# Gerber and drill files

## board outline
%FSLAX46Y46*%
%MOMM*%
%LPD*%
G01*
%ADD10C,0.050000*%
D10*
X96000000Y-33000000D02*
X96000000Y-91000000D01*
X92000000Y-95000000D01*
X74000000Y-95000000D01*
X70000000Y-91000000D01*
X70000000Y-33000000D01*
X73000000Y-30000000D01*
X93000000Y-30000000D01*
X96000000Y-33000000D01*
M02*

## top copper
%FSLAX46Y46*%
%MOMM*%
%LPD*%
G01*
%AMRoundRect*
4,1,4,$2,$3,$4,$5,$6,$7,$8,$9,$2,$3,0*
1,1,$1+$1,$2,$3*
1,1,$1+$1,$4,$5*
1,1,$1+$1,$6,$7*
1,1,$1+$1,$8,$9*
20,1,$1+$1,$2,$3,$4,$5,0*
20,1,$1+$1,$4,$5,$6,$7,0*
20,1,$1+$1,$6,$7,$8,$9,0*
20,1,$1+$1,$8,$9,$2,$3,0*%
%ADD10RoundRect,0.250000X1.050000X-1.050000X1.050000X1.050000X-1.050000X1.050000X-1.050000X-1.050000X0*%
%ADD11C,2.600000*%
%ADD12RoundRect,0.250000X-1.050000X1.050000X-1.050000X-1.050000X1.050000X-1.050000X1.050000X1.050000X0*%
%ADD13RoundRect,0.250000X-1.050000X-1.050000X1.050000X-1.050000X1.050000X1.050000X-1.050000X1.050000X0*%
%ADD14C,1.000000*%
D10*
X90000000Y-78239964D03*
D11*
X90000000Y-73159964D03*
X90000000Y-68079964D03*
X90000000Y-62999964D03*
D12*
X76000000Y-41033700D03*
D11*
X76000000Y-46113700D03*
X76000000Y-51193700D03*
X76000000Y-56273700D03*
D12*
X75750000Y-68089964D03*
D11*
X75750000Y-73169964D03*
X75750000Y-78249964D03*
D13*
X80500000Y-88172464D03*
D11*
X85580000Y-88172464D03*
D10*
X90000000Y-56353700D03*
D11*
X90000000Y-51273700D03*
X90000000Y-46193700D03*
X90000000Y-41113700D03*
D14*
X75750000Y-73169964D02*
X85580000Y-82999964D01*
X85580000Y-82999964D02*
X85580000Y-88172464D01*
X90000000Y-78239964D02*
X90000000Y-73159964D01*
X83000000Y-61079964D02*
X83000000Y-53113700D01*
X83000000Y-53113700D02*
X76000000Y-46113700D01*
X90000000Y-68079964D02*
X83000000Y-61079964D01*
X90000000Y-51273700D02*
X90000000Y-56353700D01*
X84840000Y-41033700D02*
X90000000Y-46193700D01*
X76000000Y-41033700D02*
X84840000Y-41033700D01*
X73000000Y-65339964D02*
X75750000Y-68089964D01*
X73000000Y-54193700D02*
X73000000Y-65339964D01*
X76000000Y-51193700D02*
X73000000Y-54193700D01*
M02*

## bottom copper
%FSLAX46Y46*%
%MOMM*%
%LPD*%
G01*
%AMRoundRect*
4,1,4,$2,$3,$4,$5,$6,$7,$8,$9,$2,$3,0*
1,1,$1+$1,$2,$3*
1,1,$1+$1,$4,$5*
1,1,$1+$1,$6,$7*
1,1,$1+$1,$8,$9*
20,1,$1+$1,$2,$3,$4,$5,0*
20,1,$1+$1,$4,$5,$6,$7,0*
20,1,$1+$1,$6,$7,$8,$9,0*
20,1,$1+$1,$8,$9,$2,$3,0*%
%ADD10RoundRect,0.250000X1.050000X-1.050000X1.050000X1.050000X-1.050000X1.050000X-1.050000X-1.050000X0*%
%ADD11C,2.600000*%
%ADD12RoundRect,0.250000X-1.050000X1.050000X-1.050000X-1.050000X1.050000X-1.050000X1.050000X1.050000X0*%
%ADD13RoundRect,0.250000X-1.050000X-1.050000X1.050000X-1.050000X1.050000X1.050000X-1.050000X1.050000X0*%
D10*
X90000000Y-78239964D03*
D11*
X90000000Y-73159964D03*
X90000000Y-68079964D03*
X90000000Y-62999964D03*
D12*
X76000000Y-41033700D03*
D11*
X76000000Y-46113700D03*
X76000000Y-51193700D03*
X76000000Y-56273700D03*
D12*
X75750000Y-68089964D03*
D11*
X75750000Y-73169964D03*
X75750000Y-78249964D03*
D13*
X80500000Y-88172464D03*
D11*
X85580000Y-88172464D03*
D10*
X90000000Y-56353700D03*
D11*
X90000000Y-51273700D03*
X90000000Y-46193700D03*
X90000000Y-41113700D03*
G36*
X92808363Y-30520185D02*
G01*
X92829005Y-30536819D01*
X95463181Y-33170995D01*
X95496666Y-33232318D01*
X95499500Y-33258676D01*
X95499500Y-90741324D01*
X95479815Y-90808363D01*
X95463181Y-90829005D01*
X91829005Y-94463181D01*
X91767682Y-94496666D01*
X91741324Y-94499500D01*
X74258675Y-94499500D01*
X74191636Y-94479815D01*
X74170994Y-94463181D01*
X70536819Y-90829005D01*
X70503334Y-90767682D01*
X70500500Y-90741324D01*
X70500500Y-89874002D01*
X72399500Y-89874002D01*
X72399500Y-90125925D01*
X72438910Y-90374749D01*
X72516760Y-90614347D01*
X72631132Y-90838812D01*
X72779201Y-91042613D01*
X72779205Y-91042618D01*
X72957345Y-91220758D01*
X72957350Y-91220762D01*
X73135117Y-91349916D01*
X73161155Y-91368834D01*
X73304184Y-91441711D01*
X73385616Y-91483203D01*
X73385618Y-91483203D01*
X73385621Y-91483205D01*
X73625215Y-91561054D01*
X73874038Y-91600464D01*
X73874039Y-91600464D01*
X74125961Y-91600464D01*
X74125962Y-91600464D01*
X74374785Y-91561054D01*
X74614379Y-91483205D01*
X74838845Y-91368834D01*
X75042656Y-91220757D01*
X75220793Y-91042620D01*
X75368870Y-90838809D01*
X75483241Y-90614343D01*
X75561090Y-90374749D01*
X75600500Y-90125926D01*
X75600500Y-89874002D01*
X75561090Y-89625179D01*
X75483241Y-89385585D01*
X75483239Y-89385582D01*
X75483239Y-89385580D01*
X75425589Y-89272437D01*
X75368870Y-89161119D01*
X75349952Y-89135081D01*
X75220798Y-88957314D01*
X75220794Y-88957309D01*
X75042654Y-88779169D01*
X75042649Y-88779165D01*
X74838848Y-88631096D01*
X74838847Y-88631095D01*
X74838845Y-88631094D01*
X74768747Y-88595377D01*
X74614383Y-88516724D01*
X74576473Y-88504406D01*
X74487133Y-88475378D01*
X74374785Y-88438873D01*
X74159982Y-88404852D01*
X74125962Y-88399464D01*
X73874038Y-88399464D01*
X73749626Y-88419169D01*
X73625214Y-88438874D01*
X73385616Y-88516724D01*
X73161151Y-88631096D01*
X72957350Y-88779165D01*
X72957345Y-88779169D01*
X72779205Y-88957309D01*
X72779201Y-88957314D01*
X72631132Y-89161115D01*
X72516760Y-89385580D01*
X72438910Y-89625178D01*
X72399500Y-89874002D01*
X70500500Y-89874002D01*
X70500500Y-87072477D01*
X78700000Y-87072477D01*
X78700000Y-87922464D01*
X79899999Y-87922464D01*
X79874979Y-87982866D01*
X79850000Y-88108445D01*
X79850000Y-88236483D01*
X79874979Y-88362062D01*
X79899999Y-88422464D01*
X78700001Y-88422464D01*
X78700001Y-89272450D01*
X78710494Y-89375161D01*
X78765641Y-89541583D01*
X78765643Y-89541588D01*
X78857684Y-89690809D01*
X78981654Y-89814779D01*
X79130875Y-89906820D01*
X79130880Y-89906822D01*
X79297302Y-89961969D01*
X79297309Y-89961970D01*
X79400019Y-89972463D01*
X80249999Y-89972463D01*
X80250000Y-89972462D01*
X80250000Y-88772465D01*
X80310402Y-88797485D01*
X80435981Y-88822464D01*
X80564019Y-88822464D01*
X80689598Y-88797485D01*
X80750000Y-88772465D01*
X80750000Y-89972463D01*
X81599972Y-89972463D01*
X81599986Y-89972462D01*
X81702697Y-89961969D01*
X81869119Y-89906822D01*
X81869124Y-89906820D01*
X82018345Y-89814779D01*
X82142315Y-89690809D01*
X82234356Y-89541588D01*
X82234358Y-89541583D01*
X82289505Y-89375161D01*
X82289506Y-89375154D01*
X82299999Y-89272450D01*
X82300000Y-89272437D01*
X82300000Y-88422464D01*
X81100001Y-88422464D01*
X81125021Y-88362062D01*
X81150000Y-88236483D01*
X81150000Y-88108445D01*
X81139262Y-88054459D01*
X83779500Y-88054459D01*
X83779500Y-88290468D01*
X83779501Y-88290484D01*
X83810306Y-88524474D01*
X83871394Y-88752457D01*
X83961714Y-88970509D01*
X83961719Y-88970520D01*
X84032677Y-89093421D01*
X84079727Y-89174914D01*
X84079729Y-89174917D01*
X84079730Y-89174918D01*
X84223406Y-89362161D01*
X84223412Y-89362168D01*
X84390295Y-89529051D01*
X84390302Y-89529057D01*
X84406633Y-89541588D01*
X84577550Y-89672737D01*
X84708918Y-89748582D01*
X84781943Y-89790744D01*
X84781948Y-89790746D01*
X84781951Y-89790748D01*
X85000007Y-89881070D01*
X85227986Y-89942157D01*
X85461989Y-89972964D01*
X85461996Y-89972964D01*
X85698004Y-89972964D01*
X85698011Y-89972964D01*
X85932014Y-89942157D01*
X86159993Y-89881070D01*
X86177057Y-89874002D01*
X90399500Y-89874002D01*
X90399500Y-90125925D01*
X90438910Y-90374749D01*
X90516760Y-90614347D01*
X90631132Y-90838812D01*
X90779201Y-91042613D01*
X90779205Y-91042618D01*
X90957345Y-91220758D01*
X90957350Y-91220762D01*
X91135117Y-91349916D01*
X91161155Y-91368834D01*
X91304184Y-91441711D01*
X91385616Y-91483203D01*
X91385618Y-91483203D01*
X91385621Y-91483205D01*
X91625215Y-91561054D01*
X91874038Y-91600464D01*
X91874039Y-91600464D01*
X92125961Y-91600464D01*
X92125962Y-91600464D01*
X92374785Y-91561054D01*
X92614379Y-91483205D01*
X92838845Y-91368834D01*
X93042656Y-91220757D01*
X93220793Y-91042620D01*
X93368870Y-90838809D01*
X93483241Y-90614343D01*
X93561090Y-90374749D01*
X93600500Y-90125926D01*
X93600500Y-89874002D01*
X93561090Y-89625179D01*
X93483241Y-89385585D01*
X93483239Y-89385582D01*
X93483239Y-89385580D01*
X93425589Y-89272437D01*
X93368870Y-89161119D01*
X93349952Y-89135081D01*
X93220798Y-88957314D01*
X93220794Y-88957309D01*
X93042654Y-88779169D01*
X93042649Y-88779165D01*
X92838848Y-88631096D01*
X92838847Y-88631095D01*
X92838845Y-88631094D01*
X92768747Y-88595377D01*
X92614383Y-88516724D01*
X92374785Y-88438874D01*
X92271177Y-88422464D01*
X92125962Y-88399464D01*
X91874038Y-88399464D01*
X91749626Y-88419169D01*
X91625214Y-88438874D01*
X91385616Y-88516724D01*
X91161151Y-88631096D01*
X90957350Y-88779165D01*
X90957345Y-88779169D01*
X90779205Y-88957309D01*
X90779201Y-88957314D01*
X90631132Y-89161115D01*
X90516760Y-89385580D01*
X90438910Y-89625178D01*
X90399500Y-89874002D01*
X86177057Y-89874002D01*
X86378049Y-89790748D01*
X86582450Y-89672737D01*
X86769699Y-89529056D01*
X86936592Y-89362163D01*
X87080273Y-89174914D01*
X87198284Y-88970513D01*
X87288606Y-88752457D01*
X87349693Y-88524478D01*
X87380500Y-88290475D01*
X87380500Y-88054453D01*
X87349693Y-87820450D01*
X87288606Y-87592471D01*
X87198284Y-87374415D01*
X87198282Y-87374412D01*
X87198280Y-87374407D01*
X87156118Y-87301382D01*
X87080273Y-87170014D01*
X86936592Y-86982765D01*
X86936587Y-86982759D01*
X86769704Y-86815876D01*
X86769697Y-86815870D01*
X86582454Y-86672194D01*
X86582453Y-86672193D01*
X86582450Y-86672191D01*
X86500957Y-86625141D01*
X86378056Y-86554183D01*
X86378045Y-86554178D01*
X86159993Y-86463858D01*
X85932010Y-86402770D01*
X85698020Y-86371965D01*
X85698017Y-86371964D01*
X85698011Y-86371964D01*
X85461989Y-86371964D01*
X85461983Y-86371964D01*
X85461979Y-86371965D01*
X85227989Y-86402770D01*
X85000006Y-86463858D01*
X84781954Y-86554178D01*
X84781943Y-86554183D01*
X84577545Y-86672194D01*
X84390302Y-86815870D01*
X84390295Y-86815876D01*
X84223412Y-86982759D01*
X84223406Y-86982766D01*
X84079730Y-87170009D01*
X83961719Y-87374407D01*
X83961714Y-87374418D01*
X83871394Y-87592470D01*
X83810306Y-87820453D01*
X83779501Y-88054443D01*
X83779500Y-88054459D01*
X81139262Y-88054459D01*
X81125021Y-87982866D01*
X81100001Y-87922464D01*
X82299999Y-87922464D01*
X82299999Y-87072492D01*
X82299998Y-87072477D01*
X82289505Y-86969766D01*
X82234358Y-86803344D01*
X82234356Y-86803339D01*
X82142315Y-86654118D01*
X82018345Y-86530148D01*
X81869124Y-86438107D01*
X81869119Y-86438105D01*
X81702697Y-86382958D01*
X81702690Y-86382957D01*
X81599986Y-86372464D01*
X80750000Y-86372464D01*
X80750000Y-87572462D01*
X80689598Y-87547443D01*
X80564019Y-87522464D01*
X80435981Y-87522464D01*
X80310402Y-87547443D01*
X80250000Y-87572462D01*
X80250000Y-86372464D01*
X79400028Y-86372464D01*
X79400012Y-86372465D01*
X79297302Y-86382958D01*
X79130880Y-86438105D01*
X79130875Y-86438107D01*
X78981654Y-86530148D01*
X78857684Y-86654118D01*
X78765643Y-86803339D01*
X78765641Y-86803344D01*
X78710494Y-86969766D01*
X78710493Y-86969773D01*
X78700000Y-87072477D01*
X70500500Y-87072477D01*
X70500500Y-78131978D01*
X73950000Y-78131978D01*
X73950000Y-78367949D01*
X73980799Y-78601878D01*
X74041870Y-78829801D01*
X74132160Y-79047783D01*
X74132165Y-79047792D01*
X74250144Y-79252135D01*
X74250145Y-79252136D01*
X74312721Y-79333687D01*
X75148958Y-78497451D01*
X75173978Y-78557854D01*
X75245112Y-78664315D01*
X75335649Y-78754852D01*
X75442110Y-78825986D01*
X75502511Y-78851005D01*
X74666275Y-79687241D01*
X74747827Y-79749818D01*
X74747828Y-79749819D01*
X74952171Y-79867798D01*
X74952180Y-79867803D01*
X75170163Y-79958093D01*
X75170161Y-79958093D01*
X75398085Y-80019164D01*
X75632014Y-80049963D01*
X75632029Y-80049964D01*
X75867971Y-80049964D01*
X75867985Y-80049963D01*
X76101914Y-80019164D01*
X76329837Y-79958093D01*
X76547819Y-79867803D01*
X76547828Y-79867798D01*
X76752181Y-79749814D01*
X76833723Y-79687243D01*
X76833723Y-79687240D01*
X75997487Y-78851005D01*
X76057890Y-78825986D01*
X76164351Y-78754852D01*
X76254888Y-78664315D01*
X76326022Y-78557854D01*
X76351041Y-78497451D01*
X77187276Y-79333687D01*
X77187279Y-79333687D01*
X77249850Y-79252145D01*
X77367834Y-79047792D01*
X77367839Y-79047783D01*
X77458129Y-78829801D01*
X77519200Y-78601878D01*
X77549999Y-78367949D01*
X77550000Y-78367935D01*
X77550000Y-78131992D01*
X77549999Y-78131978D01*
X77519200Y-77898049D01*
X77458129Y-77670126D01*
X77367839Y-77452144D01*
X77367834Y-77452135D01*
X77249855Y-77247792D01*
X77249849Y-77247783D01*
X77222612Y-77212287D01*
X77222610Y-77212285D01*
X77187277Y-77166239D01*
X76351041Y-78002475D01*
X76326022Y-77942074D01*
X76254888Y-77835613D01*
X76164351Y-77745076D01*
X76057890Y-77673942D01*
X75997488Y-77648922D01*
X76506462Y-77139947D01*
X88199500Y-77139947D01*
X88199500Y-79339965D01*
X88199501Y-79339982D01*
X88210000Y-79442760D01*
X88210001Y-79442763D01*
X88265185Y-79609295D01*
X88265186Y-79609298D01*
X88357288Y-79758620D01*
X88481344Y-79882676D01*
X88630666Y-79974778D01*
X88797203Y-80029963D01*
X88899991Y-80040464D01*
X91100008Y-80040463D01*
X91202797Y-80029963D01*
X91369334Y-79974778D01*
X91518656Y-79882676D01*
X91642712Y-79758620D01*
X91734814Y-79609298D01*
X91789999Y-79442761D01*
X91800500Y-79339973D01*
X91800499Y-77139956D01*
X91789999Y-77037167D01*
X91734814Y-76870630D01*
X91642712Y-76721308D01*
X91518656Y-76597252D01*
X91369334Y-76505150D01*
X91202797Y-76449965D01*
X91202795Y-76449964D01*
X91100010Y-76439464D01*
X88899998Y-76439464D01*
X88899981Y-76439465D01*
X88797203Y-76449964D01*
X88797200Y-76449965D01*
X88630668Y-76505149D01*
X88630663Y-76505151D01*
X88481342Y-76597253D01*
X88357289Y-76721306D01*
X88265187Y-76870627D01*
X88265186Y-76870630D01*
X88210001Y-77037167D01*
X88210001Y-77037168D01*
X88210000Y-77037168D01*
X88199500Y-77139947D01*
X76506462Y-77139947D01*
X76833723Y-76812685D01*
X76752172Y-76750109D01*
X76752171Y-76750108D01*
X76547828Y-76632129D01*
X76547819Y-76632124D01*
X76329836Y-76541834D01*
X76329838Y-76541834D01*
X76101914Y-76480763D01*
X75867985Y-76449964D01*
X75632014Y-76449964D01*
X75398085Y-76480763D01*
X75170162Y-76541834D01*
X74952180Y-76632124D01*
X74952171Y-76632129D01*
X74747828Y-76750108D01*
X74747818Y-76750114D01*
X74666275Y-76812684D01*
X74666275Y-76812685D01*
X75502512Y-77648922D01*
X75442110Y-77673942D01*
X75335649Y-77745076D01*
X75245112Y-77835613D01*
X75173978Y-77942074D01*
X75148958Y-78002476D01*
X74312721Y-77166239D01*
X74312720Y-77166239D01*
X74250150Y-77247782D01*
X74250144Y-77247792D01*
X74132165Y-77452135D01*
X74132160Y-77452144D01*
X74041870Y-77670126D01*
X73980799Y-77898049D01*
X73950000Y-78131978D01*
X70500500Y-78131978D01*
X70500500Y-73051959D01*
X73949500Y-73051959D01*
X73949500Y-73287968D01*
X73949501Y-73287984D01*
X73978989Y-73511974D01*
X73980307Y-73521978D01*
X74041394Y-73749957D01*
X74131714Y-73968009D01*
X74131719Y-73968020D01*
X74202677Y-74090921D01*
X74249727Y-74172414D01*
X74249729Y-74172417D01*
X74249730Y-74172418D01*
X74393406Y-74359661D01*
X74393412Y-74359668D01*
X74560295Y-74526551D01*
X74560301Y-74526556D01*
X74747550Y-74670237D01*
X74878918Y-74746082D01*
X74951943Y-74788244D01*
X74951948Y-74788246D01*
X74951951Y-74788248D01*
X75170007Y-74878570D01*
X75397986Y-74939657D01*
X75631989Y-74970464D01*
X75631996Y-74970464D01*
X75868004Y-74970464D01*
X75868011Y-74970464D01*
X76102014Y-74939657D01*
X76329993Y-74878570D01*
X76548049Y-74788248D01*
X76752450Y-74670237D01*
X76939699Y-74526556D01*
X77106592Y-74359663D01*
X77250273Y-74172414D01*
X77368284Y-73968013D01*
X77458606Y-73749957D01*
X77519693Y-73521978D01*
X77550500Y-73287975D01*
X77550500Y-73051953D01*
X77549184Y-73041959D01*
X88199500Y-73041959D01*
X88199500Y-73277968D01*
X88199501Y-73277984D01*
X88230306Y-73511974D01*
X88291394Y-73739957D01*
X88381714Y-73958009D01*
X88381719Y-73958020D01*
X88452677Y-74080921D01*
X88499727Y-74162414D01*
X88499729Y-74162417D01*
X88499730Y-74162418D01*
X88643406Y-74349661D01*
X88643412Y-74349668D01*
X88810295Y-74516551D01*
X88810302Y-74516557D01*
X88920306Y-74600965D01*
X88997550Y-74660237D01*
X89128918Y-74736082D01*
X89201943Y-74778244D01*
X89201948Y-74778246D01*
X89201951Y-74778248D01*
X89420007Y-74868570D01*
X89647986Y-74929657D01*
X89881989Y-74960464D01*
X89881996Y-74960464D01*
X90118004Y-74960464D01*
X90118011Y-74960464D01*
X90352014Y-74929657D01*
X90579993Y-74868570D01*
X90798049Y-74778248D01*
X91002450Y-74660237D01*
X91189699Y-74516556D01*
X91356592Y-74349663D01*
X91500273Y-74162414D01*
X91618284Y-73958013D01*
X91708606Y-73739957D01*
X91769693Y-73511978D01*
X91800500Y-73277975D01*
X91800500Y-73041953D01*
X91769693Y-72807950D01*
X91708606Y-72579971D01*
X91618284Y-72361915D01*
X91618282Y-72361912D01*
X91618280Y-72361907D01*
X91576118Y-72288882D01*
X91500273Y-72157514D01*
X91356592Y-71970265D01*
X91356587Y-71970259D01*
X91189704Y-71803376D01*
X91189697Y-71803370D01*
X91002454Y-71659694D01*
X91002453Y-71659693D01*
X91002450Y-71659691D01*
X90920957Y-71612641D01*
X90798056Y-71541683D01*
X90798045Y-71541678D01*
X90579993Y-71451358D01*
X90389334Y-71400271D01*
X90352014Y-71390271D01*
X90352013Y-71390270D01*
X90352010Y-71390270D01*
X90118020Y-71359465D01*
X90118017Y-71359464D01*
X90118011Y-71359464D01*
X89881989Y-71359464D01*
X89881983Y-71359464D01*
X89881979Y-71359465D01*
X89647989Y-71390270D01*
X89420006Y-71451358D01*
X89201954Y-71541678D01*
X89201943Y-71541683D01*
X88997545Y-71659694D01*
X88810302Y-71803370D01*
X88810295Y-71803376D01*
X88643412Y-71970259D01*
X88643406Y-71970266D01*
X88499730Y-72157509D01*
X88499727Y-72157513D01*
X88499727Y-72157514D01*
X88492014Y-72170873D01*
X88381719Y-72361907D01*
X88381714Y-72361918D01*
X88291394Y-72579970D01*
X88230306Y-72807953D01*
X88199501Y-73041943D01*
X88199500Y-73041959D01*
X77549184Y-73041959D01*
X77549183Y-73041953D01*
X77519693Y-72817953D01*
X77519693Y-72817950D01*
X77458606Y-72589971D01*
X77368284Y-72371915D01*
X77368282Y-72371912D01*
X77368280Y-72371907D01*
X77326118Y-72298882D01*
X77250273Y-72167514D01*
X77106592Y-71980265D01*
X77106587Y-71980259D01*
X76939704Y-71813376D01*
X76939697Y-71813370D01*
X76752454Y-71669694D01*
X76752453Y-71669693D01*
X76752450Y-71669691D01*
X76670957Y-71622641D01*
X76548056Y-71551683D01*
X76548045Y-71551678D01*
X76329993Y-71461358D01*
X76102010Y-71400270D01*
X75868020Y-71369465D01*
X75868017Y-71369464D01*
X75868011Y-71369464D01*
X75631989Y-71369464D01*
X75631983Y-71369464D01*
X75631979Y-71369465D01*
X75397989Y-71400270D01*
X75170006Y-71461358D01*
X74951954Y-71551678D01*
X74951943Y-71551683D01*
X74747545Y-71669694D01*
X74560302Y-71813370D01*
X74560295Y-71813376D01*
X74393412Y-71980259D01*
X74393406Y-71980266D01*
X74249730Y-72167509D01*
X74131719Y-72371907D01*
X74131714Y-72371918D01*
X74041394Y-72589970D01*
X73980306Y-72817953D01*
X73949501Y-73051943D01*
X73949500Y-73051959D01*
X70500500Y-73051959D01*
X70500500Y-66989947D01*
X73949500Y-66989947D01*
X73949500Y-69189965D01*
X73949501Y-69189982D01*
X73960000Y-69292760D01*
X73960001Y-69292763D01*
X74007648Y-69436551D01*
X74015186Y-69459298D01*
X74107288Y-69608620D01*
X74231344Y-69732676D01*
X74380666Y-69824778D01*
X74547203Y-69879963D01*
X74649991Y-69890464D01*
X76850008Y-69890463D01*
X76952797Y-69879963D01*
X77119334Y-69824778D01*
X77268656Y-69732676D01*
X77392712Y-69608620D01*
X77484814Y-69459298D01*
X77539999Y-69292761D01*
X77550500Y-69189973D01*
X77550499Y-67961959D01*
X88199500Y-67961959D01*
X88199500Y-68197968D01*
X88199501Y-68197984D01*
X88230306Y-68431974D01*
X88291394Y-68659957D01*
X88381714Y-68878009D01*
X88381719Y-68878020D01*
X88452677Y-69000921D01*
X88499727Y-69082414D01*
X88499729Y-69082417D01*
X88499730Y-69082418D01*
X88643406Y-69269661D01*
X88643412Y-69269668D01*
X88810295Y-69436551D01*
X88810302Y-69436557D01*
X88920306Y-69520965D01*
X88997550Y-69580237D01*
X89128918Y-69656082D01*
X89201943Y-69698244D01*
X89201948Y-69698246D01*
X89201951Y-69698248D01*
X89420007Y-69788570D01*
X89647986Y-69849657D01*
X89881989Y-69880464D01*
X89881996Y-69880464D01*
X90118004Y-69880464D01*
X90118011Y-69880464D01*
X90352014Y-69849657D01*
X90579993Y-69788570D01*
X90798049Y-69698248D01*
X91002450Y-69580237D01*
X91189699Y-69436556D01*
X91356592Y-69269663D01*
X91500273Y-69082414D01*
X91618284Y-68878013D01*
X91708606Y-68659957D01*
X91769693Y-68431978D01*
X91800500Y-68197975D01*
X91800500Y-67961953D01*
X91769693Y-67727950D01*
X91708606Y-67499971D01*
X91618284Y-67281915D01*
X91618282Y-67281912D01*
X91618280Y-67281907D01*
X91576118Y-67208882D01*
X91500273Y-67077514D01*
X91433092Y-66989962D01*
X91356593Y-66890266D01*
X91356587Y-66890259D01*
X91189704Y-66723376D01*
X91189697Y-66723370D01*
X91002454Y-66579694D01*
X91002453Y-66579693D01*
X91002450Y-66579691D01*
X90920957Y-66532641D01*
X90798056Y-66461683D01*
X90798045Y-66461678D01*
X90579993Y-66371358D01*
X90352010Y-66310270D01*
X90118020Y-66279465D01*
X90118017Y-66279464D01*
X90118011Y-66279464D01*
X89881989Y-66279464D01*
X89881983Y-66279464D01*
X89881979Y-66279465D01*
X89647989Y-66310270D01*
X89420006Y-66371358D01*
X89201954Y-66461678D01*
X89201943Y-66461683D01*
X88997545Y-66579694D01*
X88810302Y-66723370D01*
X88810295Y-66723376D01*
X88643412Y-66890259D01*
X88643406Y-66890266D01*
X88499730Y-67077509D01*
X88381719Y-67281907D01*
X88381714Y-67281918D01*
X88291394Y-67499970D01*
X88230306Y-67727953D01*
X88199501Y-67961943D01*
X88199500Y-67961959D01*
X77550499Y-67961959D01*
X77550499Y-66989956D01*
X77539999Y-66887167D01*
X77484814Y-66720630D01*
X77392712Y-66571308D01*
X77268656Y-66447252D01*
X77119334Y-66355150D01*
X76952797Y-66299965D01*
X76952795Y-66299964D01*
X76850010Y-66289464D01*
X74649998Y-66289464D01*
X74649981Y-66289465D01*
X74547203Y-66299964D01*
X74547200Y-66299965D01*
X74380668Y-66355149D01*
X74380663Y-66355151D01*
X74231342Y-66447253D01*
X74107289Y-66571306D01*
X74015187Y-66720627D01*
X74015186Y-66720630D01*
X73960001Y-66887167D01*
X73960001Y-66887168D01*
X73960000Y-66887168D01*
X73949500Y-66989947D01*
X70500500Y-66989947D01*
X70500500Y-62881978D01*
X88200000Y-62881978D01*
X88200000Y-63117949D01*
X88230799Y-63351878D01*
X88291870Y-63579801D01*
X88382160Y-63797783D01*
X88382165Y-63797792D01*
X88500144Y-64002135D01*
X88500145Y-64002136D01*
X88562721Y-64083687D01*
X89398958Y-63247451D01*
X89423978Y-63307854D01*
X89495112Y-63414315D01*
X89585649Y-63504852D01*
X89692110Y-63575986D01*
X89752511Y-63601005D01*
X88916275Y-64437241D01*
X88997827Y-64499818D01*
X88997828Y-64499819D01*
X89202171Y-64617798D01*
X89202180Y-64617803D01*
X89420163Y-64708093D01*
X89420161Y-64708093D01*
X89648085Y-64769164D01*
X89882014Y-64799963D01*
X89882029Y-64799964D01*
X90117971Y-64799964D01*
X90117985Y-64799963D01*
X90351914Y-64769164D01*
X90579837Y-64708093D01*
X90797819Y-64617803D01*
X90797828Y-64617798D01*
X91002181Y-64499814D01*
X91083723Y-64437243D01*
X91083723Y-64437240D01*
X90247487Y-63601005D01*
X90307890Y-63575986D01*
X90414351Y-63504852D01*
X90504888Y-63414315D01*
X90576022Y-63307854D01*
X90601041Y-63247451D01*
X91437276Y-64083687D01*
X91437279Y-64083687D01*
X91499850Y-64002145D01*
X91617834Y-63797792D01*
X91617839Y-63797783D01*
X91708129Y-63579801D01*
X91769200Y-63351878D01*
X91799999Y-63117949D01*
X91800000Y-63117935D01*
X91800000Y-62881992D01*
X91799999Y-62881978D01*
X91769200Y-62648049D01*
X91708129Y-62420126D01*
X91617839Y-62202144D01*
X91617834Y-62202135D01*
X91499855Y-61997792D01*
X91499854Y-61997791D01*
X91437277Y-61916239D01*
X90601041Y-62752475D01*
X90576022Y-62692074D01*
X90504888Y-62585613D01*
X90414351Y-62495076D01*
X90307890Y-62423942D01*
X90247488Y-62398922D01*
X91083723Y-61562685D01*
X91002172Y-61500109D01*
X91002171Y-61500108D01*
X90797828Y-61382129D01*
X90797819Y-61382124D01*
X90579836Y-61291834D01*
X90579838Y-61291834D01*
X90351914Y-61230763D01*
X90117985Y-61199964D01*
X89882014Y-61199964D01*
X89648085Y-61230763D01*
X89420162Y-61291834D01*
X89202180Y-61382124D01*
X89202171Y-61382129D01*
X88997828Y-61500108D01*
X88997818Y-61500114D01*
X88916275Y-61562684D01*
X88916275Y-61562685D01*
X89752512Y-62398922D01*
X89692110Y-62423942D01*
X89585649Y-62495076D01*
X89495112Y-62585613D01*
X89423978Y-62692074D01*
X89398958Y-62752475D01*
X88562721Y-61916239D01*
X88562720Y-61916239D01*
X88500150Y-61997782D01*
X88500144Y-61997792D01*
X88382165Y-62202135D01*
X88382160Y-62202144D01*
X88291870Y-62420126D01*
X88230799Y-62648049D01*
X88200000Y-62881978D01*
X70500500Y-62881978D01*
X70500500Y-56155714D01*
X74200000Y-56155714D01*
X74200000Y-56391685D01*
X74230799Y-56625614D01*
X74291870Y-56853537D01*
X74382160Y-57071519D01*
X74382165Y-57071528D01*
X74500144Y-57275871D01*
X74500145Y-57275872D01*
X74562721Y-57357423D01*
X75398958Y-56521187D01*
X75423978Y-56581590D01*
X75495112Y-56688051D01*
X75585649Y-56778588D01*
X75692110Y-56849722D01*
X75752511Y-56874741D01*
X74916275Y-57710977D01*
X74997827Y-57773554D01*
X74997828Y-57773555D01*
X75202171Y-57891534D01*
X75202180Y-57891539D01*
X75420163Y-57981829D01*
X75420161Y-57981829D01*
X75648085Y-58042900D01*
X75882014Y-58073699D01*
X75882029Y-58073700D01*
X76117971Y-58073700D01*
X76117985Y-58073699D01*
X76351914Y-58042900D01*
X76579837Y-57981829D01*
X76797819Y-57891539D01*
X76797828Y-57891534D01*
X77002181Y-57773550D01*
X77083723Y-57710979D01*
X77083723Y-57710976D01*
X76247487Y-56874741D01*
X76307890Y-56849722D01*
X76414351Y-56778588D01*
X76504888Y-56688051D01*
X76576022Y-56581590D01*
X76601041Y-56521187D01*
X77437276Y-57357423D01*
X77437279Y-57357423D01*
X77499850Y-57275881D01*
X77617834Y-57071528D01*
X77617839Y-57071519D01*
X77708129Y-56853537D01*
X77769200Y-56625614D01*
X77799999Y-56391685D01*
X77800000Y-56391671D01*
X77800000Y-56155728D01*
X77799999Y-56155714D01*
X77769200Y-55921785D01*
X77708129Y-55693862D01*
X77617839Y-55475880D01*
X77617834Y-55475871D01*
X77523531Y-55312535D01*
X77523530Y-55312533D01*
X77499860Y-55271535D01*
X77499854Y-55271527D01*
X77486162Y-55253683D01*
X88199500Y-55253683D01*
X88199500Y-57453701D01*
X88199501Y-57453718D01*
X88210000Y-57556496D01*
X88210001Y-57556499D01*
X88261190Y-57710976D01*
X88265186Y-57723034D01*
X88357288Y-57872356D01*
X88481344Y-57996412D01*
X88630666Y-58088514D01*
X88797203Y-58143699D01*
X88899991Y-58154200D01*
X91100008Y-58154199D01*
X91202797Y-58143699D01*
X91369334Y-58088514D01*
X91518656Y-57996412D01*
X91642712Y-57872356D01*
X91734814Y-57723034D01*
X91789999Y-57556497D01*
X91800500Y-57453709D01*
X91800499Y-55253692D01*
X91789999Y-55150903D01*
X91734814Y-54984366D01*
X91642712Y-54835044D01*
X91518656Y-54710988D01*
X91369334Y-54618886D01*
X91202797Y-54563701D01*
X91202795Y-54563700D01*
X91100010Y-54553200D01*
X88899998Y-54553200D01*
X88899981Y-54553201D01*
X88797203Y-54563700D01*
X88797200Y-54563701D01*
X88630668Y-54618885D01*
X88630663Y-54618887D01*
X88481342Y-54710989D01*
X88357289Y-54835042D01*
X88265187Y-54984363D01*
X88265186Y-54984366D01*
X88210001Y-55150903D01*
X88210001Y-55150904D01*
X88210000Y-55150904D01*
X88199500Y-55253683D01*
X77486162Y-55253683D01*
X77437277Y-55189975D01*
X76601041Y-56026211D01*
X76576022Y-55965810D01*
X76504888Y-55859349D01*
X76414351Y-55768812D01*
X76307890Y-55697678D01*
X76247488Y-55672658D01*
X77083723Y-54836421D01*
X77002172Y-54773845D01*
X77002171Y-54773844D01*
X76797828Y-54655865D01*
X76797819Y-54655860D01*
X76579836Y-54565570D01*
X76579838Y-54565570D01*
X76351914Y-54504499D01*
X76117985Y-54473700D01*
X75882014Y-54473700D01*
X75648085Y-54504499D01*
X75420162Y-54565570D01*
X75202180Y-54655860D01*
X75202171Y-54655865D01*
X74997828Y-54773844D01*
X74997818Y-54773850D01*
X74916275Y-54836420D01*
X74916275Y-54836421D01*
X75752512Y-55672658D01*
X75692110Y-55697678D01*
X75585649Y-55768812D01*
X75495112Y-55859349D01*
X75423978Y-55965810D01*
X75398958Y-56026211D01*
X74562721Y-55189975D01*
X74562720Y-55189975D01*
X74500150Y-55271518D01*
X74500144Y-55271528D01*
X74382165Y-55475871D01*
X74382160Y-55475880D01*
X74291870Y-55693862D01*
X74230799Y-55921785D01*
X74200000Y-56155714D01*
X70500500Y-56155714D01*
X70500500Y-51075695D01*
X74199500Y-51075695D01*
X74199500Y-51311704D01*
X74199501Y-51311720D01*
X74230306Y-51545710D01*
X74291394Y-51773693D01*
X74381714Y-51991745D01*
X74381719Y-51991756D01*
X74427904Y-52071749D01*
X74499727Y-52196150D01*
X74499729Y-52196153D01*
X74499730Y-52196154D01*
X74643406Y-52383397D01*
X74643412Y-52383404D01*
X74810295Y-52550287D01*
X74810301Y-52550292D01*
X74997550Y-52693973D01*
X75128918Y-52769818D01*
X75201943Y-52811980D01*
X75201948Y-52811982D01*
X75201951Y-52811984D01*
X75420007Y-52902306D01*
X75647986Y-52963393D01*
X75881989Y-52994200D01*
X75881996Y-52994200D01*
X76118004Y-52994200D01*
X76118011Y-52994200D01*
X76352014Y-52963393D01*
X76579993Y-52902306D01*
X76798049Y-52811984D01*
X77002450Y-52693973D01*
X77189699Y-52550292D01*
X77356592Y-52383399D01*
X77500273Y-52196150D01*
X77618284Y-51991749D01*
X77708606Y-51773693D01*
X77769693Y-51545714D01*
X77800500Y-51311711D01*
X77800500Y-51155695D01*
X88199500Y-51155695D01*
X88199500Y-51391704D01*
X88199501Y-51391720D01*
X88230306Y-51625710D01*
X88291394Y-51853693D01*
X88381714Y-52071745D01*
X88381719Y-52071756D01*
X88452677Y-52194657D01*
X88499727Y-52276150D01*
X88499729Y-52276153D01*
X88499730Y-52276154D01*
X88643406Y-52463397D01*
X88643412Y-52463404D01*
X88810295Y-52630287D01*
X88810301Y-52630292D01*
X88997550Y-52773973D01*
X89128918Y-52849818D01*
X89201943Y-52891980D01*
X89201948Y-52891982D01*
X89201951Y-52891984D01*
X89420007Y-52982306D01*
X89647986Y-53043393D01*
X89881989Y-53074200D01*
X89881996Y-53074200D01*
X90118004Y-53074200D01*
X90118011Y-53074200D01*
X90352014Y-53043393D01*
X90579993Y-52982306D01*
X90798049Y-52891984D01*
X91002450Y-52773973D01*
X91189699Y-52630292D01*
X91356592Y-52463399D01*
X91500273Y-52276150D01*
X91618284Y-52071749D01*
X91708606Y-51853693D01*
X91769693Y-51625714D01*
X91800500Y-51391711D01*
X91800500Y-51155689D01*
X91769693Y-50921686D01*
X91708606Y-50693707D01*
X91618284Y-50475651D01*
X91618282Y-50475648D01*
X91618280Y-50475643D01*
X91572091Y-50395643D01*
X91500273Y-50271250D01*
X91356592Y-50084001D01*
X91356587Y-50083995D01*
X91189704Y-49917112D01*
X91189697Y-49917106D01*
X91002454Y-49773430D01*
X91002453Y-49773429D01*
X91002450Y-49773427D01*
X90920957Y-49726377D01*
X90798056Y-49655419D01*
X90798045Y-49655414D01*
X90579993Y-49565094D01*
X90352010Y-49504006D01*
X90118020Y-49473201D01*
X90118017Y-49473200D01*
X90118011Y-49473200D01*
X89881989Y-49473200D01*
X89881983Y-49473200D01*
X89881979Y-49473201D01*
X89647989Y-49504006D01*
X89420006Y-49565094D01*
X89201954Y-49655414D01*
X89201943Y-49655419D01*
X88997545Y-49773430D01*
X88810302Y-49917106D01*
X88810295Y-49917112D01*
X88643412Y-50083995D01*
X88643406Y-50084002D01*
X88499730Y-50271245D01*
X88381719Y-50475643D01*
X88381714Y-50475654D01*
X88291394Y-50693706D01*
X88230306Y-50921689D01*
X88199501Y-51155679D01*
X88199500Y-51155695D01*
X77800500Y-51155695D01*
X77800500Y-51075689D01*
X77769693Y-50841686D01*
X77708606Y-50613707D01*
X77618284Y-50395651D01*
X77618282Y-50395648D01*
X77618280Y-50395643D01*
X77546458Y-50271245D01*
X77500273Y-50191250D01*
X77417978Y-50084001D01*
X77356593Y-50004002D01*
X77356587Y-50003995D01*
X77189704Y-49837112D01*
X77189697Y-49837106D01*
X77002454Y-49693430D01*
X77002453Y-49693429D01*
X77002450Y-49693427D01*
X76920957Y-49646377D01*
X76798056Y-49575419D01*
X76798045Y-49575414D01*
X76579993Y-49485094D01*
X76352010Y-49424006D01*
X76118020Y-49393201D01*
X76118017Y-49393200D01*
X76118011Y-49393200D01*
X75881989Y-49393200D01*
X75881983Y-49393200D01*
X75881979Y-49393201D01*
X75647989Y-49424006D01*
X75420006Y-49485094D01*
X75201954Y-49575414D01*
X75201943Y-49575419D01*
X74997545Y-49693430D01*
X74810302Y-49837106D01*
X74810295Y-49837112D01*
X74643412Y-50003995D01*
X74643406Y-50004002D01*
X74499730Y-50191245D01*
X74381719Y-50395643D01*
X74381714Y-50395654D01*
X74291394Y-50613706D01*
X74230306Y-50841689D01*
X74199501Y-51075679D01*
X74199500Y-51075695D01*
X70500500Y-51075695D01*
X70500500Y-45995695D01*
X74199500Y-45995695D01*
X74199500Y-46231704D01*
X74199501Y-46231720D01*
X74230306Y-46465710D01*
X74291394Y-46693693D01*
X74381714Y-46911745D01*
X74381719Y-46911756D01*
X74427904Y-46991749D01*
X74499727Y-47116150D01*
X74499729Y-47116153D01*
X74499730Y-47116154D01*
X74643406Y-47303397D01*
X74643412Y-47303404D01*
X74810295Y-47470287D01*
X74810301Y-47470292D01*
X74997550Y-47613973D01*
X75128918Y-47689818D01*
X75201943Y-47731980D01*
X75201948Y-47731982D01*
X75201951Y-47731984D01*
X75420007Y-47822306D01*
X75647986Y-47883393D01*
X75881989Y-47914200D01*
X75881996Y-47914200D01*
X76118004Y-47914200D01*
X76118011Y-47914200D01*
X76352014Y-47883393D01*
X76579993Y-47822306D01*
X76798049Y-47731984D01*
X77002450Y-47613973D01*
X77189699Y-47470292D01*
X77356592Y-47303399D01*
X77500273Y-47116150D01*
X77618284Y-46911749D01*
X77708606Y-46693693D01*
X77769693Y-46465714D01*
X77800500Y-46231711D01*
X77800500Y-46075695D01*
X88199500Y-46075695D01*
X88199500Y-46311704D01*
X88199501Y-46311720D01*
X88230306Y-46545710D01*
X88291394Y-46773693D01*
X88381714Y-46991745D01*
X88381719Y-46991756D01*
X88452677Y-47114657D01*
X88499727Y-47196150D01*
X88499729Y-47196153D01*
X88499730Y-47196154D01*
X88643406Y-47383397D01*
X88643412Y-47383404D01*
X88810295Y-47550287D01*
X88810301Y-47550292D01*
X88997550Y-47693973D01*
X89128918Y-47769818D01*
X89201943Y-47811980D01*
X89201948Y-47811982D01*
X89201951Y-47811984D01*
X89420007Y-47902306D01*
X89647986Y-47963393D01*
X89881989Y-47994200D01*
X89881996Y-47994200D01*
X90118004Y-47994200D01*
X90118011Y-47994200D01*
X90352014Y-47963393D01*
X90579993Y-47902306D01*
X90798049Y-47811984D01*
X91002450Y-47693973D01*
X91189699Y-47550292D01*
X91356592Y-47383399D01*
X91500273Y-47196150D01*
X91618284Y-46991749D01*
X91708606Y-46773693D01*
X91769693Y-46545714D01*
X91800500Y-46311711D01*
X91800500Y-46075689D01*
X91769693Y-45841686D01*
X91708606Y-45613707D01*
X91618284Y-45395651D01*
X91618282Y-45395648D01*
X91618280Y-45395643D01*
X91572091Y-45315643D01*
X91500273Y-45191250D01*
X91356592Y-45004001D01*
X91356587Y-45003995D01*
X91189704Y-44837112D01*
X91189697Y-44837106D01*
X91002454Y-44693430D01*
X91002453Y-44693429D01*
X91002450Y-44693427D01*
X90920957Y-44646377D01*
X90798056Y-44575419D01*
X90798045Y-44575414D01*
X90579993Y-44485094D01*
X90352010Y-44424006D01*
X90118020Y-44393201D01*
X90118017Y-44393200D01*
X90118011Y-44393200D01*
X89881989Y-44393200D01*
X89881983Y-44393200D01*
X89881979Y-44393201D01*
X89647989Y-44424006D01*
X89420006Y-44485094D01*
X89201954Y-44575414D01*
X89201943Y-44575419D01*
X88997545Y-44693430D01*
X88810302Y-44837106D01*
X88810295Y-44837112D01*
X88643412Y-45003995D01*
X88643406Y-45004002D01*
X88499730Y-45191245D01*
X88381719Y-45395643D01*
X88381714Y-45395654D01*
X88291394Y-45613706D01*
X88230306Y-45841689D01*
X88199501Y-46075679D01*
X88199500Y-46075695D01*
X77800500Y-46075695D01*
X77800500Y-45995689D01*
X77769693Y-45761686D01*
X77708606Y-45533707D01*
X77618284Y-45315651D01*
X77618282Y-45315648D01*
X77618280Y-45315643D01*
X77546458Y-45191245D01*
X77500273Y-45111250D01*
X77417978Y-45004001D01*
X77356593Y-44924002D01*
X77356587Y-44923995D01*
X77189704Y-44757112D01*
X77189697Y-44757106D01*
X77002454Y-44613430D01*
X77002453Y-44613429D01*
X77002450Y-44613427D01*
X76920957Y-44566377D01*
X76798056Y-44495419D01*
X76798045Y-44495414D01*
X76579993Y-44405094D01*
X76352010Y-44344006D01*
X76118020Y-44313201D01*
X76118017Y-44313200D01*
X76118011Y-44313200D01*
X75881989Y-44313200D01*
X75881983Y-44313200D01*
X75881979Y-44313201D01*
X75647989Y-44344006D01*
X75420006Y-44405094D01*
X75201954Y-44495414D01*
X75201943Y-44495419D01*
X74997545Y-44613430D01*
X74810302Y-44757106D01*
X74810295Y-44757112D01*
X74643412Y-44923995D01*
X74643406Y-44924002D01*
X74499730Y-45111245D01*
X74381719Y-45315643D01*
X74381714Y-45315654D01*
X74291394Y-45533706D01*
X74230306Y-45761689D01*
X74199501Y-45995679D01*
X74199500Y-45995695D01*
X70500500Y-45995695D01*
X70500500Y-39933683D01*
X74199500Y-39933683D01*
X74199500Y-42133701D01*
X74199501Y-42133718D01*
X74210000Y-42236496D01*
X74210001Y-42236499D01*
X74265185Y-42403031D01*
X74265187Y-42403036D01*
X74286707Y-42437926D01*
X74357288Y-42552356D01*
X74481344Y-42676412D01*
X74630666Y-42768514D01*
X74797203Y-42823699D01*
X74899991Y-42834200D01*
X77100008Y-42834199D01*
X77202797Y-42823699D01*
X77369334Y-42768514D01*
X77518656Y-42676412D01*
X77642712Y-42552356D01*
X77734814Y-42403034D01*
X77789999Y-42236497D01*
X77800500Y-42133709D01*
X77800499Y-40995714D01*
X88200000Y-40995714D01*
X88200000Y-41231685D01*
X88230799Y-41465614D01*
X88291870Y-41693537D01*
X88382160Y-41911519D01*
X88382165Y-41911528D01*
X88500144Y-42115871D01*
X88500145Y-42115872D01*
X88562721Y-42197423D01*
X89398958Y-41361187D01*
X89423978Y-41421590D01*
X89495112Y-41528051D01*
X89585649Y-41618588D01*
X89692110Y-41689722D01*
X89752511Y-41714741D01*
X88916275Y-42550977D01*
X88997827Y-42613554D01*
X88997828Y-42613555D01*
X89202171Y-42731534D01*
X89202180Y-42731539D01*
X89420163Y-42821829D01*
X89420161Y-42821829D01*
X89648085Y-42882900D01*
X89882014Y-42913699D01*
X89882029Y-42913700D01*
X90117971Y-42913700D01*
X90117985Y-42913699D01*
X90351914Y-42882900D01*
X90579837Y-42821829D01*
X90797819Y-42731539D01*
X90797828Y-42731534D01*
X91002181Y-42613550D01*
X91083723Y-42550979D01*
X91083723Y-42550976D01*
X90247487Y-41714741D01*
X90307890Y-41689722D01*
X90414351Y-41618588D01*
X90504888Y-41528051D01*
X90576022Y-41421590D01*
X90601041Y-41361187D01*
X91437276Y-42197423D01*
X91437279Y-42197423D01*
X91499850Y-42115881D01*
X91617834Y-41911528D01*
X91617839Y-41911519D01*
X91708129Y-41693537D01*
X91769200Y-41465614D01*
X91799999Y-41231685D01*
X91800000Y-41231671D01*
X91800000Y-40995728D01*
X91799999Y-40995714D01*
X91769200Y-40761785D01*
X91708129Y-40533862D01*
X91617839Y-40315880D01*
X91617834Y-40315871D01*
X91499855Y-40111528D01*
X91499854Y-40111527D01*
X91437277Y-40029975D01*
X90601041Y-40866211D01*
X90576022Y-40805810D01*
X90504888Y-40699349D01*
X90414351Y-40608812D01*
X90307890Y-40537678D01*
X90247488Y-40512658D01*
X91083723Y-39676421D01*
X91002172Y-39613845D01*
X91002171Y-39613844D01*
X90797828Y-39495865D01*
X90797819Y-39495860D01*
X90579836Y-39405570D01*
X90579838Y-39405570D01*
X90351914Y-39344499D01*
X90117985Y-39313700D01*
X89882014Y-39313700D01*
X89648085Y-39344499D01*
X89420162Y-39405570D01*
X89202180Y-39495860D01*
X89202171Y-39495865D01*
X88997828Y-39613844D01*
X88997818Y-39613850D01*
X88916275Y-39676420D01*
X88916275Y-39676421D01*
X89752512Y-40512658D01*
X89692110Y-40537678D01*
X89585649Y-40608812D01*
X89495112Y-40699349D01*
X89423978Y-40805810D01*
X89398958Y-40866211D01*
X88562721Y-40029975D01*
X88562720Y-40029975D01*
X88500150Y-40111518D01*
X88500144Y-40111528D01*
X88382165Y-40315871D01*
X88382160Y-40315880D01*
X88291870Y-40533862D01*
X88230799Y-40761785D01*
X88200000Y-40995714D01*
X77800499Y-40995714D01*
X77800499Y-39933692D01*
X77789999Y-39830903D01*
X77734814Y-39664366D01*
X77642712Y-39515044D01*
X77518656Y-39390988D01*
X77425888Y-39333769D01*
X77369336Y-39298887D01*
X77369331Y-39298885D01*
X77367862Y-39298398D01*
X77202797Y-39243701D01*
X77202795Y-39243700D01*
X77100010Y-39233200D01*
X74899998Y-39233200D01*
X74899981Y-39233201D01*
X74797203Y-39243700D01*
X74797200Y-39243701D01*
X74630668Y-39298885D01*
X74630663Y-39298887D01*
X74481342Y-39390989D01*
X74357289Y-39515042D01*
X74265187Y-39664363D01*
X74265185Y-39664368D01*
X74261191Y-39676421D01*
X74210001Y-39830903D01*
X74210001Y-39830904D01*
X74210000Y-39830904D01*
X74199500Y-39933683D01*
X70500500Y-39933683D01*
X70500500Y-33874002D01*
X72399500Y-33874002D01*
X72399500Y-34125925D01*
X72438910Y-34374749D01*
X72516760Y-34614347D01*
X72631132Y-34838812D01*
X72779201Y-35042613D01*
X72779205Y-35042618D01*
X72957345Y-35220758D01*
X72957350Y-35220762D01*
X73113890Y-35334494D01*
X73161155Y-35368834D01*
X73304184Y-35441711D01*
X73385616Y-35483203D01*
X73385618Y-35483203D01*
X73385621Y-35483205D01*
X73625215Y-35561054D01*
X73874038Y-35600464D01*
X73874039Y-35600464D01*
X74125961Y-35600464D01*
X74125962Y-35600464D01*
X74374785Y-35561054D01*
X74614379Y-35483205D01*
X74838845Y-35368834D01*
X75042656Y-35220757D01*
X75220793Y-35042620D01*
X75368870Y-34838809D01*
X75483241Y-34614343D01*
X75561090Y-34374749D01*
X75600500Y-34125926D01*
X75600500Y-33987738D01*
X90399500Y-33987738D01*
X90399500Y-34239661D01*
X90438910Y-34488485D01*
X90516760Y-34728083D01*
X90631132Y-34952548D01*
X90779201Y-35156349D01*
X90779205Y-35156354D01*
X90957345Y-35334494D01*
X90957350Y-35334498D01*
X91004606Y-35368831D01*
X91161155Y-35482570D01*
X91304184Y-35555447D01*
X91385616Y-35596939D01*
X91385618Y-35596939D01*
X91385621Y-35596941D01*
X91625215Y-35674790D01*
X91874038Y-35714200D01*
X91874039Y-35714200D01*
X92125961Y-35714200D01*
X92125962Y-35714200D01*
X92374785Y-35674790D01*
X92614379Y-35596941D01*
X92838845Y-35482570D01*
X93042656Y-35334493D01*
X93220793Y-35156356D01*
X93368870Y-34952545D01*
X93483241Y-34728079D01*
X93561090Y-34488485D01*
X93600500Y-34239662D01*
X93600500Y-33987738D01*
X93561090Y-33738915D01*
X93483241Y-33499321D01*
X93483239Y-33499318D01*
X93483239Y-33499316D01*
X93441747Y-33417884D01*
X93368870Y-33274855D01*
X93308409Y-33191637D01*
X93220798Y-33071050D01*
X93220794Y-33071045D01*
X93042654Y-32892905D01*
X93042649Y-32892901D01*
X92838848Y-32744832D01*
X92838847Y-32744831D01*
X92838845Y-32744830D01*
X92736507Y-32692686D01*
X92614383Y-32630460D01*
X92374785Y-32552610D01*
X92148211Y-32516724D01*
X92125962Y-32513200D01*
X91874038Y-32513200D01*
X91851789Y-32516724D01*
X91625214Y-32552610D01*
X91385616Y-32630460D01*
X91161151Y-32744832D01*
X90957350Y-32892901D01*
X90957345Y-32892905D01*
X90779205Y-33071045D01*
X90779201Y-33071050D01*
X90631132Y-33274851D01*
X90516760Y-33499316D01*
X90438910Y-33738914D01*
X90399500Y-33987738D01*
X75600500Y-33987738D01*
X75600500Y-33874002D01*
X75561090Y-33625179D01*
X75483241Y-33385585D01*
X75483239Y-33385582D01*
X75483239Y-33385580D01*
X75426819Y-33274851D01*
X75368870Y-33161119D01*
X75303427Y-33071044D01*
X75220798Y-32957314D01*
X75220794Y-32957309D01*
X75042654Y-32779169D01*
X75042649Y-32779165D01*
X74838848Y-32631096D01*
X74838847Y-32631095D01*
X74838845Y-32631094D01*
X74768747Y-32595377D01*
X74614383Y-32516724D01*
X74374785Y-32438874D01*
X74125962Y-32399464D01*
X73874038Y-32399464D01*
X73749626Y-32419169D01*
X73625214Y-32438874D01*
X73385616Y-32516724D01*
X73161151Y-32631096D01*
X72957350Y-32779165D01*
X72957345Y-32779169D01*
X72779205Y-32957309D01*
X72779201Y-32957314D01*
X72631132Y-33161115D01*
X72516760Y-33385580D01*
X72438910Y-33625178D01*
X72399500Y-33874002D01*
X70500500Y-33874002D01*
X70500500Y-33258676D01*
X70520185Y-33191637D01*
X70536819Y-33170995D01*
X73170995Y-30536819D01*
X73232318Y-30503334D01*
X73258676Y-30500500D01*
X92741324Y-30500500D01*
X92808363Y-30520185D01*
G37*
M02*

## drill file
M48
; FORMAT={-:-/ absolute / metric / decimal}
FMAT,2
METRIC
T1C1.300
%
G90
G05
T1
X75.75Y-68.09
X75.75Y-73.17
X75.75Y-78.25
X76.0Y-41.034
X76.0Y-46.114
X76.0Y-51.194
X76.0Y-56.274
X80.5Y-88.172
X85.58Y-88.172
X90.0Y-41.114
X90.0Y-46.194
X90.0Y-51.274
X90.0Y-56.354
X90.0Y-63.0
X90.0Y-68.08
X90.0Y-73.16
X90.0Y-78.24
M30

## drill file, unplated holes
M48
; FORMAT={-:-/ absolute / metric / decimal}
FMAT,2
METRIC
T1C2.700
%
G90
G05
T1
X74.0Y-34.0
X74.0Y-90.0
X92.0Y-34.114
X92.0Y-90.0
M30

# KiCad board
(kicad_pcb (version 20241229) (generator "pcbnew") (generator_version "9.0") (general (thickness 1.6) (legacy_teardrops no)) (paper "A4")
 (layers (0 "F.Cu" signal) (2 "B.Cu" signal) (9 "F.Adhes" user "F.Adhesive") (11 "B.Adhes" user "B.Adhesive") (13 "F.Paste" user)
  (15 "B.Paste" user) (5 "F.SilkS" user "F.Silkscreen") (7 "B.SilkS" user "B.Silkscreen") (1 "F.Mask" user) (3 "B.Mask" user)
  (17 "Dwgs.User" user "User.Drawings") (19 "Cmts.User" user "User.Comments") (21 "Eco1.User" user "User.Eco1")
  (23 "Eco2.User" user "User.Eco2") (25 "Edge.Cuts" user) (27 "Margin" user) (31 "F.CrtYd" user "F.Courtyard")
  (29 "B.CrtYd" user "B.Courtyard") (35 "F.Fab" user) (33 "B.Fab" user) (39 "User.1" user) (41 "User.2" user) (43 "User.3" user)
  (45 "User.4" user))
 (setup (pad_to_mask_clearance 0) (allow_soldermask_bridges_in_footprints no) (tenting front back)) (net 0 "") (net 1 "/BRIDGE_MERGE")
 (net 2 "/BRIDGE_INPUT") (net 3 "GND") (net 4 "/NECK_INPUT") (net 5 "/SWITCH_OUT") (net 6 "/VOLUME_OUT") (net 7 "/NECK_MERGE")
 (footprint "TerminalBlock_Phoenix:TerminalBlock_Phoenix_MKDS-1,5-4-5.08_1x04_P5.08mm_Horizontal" (layer "F.Cu") (at 90 78.239964 90)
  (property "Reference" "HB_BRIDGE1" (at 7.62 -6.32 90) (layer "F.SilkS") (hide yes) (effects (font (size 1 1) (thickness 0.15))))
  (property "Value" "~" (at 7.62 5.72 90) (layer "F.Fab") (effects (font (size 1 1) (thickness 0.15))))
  (pad "1" thru_hole roundrect (at 0 0 90) (size 2.6 2.6) (drill 1.3) (layers "*.Cu" "*.Mask") (remove_unused_layers no)
   (roundrect_rratio 0.096154) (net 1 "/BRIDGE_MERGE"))
  (pad "2" thru_hole circle (at 5.08 0 90) (size 2.6 2.6) (drill 1.3) (layers "*.Cu" "*.Mask") (remove_unused_layers no)
   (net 1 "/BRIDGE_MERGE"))
  (pad "3" thru_hole circle (at 10.16 0 90) (size 2.6 2.6) (drill 1.3) (layers "*.Cu" "*.Mask") (remove_unused_layers no)
   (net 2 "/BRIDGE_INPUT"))
  (pad "4" thru_hole circle (at 15.24 0 90) (size 2.6 2.6) (drill 1.3) (layers "*.Cu" "*.Mask") (remove_unused_layers no) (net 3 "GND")))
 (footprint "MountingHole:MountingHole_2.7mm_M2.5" (layer "F.Cu") (at 74 89.999964 180)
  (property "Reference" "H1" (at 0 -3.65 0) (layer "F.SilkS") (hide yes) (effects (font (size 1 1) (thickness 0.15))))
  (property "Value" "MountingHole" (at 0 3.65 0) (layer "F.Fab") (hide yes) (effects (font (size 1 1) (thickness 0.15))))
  (pad "" np_thru_hole circle (at 0 0 180) (size 2.7 2.7) (drill 2.7) (layers "*.Cu" "*.Mask")))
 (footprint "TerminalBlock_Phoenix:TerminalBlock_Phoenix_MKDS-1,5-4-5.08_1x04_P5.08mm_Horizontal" (layer "F.Cu") (at 76 41.0337 -90)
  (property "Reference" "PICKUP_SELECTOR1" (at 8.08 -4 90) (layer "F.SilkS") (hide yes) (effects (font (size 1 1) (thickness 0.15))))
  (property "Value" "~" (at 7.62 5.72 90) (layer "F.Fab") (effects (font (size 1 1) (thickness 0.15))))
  (pad "1" thru_hole roundrect (at 0 0 270) (size 2.6 2.6) (drill 1.3) (layers "*.Cu" "*.Mask") (remove_unused_layers no)
   (roundrect_rratio 0.096154) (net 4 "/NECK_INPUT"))
  (pad "2" thru_hole circle (at 5.08 0 270) (size 2.6 2.6) (drill 1.3) (layers "*.Cu" "*.Mask") (remove_unused_layers no)
   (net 2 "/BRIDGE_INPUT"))
  (pad "3" thru_hole circle (at 10.16 0 270) (size 2.6 2.6) (drill 1.3) (layers "*.Cu" "*.Mask") (remove_unused_layers no)
   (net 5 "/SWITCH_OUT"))
  (pad "4" thru_hole circle (at 15.24 0 270) (size 2.6 2.6) (drill 1.3) (layers "*.Cu" "*.Mask") (remove_unused_layers no) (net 3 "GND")))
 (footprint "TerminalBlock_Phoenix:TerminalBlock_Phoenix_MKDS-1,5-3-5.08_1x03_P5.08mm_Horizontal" (layer "F.Cu") (at 75.75 68.089964 -90)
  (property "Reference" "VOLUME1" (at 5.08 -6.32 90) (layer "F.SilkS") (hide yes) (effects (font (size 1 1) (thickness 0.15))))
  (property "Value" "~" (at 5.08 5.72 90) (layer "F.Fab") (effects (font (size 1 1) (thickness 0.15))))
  (pad "1" thru_hole roundrect (at 0 0 270) (size 2.6 2.6) (drill 1.3) (layers "*.Cu" "*.Mask") (remove_unused_layers no)
   (roundrect_rratio 0.096154) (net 5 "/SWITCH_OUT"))
  (pad "2" thru_hole circle (at 5.08 0 270) (size 2.6 2.6) (drill 1.3) (layers "*.Cu" "*.Mask") (remove_unused_layers no)
   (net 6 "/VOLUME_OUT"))
  (pad "3" thru_hole circle (at 10.16 0 270) (size 2.6 2.6) (drill 1.3) (layers "*.Cu" "*.Mask") (remove_unused_layers no) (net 3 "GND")))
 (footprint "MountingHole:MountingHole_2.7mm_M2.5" (layer "F.Cu") (at 74 33.999964 180)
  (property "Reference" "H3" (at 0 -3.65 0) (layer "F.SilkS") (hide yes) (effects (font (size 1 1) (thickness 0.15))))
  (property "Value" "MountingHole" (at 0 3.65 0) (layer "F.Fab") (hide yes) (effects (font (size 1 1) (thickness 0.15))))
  (pad "" np_thru_hole circle (at 0 0 180) (size 2.7 2.7) (drill 2.7) (layers "*.Cu" "*.Mask")))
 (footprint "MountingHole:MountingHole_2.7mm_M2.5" (layer "F.Cu") (at 92 34.1137 180)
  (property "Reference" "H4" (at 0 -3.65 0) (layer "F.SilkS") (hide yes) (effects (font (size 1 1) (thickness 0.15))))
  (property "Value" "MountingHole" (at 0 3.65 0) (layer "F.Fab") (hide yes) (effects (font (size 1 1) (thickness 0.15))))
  (pad "" np_thru_hole circle (at 0 0 180) (size 2.7 2.7) (drill 2.7) (layers "*.Cu" "*.Mask")))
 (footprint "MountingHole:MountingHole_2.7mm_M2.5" (layer "F.Cu") (at 92 89.999964 180)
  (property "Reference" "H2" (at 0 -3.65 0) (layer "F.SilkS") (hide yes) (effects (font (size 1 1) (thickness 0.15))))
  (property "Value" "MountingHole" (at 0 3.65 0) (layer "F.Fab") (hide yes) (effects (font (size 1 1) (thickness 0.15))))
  (pad "" np_thru_hole circle (at 0 0 180) (size 2.7 2.7) (drill 2.7) (layers "*.Cu" "*.Mask")))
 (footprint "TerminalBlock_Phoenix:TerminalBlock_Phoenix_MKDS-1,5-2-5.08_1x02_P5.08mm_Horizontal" (layer "F.Cu") (at 80.5 88.172464)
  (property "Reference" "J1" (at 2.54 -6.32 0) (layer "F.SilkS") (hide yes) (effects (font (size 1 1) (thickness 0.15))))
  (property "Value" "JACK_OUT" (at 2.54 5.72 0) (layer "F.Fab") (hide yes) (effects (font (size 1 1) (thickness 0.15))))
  (pad "1" thru_hole roundrect (at 0 0) (size 2.6 2.6) (drill 1.3) (layers "*.Cu" "*.Mask") (remove_unused_layers no)
   (roundrect_rratio 0.096154) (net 3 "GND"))
  (pad "2" thru_hole circle (at 5.08 0) (size 2.6 2.6) (drill 1.3) (layers "*.Cu" "*.Mask") (remove_unused_layers no) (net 6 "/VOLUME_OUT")))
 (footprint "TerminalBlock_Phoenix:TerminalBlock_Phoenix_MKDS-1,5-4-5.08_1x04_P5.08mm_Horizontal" (layer "F.Cu") (at 90 56.3537 90)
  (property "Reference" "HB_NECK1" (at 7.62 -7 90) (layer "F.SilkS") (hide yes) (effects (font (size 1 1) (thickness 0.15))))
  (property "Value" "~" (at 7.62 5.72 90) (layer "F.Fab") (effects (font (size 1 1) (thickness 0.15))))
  (pad "1" thru_hole roundrect (at 0 0 90) (size 2.6 2.6) (drill 1.3) (layers "*.Cu" "*.Mask") (remove_unused_layers no)
   (roundrect_rratio 0.096154) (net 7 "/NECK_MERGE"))
  (pad "2" thru_hole circle (at 5.08 0 90) (size 2.6 2.6) (drill 1.3) (layers "*.Cu" "*.Mask") (remove_unused_layers no)
   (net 7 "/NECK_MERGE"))
  (pad "3" thru_hole circle (at 10.16 0 90) (size 2.6 2.6) (drill 1.3) (layers "*.Cu" "*.Mask") (remove_unused_layers no)
   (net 4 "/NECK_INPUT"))
  (pad "4" thru_hole circle (at 15.24 0 90) (size 2.6 2.6) (drill 1.3) (layers "*.Cu" "*.Mask") (remove_unused_layers no) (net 3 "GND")))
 (gr_poly
  (pts (xy 70 91) (xy 74 95) (xy 92 95) (xy 96 91) (xy 96 33) (xy 93 30) (xy 73 30) (xy 70 33)) (stroke (width 0.05) (type solid)) (fill no)
  (layer "Edge.Cuts"))
 (segment (start 75.75 73.169964) (end 85.58 82.999964) (width 1) (layer "F.Cu") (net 6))
 (segment (start 85.58 82.999964) (end 85.58 88.172464) (width 1) (layer "F.Cu") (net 6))
 (segment (start 90 78.239964) (end 90 73.159964) (width 1) (layer "F.Cu") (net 1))
 (segment (start 83 61.079964) (end 83 53.1137) (width 1) (layer "F.Cu") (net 2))
 (segment (start 83 53.1137) (end 76 46.1137) (width 1) (layer "F.Cu") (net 2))
 (segment (start 90 68.079964) (end 83 61.079964) (width 1) (layer "F.Cu") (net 2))
 (segment (start 90 51.2737) (end 90 56.3537) (width 1) (layer "F.Cu") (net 7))
 (segment (start 84.84 41.0337) (end 90 46.1937) (width 1) (layer "F.Cu") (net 4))
 (segment (start 76 41.0337) (end 84.84 41.0337) (width 1) (layer "F.Cu") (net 4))
 (segment (start 73 65.339964) (end 75.75 68.089964) (width 1) (layer "F.Cu") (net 5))
 (segment (start 73 54.1937) (end 73 65.339964) (width 1) (layer "F.Cu") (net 5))
 (segment (start 76 51.1937) (end 73 54.1937) (width 1) (layer "F.Cu") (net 5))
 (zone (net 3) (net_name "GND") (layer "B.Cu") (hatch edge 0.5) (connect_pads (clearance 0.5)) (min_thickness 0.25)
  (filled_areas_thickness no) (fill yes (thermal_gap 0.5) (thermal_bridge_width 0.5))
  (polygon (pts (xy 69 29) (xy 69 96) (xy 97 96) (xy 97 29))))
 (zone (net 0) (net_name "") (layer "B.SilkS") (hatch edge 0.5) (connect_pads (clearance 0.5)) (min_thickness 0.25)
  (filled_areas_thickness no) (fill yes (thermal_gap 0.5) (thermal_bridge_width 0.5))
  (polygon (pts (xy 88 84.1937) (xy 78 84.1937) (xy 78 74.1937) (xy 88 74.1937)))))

